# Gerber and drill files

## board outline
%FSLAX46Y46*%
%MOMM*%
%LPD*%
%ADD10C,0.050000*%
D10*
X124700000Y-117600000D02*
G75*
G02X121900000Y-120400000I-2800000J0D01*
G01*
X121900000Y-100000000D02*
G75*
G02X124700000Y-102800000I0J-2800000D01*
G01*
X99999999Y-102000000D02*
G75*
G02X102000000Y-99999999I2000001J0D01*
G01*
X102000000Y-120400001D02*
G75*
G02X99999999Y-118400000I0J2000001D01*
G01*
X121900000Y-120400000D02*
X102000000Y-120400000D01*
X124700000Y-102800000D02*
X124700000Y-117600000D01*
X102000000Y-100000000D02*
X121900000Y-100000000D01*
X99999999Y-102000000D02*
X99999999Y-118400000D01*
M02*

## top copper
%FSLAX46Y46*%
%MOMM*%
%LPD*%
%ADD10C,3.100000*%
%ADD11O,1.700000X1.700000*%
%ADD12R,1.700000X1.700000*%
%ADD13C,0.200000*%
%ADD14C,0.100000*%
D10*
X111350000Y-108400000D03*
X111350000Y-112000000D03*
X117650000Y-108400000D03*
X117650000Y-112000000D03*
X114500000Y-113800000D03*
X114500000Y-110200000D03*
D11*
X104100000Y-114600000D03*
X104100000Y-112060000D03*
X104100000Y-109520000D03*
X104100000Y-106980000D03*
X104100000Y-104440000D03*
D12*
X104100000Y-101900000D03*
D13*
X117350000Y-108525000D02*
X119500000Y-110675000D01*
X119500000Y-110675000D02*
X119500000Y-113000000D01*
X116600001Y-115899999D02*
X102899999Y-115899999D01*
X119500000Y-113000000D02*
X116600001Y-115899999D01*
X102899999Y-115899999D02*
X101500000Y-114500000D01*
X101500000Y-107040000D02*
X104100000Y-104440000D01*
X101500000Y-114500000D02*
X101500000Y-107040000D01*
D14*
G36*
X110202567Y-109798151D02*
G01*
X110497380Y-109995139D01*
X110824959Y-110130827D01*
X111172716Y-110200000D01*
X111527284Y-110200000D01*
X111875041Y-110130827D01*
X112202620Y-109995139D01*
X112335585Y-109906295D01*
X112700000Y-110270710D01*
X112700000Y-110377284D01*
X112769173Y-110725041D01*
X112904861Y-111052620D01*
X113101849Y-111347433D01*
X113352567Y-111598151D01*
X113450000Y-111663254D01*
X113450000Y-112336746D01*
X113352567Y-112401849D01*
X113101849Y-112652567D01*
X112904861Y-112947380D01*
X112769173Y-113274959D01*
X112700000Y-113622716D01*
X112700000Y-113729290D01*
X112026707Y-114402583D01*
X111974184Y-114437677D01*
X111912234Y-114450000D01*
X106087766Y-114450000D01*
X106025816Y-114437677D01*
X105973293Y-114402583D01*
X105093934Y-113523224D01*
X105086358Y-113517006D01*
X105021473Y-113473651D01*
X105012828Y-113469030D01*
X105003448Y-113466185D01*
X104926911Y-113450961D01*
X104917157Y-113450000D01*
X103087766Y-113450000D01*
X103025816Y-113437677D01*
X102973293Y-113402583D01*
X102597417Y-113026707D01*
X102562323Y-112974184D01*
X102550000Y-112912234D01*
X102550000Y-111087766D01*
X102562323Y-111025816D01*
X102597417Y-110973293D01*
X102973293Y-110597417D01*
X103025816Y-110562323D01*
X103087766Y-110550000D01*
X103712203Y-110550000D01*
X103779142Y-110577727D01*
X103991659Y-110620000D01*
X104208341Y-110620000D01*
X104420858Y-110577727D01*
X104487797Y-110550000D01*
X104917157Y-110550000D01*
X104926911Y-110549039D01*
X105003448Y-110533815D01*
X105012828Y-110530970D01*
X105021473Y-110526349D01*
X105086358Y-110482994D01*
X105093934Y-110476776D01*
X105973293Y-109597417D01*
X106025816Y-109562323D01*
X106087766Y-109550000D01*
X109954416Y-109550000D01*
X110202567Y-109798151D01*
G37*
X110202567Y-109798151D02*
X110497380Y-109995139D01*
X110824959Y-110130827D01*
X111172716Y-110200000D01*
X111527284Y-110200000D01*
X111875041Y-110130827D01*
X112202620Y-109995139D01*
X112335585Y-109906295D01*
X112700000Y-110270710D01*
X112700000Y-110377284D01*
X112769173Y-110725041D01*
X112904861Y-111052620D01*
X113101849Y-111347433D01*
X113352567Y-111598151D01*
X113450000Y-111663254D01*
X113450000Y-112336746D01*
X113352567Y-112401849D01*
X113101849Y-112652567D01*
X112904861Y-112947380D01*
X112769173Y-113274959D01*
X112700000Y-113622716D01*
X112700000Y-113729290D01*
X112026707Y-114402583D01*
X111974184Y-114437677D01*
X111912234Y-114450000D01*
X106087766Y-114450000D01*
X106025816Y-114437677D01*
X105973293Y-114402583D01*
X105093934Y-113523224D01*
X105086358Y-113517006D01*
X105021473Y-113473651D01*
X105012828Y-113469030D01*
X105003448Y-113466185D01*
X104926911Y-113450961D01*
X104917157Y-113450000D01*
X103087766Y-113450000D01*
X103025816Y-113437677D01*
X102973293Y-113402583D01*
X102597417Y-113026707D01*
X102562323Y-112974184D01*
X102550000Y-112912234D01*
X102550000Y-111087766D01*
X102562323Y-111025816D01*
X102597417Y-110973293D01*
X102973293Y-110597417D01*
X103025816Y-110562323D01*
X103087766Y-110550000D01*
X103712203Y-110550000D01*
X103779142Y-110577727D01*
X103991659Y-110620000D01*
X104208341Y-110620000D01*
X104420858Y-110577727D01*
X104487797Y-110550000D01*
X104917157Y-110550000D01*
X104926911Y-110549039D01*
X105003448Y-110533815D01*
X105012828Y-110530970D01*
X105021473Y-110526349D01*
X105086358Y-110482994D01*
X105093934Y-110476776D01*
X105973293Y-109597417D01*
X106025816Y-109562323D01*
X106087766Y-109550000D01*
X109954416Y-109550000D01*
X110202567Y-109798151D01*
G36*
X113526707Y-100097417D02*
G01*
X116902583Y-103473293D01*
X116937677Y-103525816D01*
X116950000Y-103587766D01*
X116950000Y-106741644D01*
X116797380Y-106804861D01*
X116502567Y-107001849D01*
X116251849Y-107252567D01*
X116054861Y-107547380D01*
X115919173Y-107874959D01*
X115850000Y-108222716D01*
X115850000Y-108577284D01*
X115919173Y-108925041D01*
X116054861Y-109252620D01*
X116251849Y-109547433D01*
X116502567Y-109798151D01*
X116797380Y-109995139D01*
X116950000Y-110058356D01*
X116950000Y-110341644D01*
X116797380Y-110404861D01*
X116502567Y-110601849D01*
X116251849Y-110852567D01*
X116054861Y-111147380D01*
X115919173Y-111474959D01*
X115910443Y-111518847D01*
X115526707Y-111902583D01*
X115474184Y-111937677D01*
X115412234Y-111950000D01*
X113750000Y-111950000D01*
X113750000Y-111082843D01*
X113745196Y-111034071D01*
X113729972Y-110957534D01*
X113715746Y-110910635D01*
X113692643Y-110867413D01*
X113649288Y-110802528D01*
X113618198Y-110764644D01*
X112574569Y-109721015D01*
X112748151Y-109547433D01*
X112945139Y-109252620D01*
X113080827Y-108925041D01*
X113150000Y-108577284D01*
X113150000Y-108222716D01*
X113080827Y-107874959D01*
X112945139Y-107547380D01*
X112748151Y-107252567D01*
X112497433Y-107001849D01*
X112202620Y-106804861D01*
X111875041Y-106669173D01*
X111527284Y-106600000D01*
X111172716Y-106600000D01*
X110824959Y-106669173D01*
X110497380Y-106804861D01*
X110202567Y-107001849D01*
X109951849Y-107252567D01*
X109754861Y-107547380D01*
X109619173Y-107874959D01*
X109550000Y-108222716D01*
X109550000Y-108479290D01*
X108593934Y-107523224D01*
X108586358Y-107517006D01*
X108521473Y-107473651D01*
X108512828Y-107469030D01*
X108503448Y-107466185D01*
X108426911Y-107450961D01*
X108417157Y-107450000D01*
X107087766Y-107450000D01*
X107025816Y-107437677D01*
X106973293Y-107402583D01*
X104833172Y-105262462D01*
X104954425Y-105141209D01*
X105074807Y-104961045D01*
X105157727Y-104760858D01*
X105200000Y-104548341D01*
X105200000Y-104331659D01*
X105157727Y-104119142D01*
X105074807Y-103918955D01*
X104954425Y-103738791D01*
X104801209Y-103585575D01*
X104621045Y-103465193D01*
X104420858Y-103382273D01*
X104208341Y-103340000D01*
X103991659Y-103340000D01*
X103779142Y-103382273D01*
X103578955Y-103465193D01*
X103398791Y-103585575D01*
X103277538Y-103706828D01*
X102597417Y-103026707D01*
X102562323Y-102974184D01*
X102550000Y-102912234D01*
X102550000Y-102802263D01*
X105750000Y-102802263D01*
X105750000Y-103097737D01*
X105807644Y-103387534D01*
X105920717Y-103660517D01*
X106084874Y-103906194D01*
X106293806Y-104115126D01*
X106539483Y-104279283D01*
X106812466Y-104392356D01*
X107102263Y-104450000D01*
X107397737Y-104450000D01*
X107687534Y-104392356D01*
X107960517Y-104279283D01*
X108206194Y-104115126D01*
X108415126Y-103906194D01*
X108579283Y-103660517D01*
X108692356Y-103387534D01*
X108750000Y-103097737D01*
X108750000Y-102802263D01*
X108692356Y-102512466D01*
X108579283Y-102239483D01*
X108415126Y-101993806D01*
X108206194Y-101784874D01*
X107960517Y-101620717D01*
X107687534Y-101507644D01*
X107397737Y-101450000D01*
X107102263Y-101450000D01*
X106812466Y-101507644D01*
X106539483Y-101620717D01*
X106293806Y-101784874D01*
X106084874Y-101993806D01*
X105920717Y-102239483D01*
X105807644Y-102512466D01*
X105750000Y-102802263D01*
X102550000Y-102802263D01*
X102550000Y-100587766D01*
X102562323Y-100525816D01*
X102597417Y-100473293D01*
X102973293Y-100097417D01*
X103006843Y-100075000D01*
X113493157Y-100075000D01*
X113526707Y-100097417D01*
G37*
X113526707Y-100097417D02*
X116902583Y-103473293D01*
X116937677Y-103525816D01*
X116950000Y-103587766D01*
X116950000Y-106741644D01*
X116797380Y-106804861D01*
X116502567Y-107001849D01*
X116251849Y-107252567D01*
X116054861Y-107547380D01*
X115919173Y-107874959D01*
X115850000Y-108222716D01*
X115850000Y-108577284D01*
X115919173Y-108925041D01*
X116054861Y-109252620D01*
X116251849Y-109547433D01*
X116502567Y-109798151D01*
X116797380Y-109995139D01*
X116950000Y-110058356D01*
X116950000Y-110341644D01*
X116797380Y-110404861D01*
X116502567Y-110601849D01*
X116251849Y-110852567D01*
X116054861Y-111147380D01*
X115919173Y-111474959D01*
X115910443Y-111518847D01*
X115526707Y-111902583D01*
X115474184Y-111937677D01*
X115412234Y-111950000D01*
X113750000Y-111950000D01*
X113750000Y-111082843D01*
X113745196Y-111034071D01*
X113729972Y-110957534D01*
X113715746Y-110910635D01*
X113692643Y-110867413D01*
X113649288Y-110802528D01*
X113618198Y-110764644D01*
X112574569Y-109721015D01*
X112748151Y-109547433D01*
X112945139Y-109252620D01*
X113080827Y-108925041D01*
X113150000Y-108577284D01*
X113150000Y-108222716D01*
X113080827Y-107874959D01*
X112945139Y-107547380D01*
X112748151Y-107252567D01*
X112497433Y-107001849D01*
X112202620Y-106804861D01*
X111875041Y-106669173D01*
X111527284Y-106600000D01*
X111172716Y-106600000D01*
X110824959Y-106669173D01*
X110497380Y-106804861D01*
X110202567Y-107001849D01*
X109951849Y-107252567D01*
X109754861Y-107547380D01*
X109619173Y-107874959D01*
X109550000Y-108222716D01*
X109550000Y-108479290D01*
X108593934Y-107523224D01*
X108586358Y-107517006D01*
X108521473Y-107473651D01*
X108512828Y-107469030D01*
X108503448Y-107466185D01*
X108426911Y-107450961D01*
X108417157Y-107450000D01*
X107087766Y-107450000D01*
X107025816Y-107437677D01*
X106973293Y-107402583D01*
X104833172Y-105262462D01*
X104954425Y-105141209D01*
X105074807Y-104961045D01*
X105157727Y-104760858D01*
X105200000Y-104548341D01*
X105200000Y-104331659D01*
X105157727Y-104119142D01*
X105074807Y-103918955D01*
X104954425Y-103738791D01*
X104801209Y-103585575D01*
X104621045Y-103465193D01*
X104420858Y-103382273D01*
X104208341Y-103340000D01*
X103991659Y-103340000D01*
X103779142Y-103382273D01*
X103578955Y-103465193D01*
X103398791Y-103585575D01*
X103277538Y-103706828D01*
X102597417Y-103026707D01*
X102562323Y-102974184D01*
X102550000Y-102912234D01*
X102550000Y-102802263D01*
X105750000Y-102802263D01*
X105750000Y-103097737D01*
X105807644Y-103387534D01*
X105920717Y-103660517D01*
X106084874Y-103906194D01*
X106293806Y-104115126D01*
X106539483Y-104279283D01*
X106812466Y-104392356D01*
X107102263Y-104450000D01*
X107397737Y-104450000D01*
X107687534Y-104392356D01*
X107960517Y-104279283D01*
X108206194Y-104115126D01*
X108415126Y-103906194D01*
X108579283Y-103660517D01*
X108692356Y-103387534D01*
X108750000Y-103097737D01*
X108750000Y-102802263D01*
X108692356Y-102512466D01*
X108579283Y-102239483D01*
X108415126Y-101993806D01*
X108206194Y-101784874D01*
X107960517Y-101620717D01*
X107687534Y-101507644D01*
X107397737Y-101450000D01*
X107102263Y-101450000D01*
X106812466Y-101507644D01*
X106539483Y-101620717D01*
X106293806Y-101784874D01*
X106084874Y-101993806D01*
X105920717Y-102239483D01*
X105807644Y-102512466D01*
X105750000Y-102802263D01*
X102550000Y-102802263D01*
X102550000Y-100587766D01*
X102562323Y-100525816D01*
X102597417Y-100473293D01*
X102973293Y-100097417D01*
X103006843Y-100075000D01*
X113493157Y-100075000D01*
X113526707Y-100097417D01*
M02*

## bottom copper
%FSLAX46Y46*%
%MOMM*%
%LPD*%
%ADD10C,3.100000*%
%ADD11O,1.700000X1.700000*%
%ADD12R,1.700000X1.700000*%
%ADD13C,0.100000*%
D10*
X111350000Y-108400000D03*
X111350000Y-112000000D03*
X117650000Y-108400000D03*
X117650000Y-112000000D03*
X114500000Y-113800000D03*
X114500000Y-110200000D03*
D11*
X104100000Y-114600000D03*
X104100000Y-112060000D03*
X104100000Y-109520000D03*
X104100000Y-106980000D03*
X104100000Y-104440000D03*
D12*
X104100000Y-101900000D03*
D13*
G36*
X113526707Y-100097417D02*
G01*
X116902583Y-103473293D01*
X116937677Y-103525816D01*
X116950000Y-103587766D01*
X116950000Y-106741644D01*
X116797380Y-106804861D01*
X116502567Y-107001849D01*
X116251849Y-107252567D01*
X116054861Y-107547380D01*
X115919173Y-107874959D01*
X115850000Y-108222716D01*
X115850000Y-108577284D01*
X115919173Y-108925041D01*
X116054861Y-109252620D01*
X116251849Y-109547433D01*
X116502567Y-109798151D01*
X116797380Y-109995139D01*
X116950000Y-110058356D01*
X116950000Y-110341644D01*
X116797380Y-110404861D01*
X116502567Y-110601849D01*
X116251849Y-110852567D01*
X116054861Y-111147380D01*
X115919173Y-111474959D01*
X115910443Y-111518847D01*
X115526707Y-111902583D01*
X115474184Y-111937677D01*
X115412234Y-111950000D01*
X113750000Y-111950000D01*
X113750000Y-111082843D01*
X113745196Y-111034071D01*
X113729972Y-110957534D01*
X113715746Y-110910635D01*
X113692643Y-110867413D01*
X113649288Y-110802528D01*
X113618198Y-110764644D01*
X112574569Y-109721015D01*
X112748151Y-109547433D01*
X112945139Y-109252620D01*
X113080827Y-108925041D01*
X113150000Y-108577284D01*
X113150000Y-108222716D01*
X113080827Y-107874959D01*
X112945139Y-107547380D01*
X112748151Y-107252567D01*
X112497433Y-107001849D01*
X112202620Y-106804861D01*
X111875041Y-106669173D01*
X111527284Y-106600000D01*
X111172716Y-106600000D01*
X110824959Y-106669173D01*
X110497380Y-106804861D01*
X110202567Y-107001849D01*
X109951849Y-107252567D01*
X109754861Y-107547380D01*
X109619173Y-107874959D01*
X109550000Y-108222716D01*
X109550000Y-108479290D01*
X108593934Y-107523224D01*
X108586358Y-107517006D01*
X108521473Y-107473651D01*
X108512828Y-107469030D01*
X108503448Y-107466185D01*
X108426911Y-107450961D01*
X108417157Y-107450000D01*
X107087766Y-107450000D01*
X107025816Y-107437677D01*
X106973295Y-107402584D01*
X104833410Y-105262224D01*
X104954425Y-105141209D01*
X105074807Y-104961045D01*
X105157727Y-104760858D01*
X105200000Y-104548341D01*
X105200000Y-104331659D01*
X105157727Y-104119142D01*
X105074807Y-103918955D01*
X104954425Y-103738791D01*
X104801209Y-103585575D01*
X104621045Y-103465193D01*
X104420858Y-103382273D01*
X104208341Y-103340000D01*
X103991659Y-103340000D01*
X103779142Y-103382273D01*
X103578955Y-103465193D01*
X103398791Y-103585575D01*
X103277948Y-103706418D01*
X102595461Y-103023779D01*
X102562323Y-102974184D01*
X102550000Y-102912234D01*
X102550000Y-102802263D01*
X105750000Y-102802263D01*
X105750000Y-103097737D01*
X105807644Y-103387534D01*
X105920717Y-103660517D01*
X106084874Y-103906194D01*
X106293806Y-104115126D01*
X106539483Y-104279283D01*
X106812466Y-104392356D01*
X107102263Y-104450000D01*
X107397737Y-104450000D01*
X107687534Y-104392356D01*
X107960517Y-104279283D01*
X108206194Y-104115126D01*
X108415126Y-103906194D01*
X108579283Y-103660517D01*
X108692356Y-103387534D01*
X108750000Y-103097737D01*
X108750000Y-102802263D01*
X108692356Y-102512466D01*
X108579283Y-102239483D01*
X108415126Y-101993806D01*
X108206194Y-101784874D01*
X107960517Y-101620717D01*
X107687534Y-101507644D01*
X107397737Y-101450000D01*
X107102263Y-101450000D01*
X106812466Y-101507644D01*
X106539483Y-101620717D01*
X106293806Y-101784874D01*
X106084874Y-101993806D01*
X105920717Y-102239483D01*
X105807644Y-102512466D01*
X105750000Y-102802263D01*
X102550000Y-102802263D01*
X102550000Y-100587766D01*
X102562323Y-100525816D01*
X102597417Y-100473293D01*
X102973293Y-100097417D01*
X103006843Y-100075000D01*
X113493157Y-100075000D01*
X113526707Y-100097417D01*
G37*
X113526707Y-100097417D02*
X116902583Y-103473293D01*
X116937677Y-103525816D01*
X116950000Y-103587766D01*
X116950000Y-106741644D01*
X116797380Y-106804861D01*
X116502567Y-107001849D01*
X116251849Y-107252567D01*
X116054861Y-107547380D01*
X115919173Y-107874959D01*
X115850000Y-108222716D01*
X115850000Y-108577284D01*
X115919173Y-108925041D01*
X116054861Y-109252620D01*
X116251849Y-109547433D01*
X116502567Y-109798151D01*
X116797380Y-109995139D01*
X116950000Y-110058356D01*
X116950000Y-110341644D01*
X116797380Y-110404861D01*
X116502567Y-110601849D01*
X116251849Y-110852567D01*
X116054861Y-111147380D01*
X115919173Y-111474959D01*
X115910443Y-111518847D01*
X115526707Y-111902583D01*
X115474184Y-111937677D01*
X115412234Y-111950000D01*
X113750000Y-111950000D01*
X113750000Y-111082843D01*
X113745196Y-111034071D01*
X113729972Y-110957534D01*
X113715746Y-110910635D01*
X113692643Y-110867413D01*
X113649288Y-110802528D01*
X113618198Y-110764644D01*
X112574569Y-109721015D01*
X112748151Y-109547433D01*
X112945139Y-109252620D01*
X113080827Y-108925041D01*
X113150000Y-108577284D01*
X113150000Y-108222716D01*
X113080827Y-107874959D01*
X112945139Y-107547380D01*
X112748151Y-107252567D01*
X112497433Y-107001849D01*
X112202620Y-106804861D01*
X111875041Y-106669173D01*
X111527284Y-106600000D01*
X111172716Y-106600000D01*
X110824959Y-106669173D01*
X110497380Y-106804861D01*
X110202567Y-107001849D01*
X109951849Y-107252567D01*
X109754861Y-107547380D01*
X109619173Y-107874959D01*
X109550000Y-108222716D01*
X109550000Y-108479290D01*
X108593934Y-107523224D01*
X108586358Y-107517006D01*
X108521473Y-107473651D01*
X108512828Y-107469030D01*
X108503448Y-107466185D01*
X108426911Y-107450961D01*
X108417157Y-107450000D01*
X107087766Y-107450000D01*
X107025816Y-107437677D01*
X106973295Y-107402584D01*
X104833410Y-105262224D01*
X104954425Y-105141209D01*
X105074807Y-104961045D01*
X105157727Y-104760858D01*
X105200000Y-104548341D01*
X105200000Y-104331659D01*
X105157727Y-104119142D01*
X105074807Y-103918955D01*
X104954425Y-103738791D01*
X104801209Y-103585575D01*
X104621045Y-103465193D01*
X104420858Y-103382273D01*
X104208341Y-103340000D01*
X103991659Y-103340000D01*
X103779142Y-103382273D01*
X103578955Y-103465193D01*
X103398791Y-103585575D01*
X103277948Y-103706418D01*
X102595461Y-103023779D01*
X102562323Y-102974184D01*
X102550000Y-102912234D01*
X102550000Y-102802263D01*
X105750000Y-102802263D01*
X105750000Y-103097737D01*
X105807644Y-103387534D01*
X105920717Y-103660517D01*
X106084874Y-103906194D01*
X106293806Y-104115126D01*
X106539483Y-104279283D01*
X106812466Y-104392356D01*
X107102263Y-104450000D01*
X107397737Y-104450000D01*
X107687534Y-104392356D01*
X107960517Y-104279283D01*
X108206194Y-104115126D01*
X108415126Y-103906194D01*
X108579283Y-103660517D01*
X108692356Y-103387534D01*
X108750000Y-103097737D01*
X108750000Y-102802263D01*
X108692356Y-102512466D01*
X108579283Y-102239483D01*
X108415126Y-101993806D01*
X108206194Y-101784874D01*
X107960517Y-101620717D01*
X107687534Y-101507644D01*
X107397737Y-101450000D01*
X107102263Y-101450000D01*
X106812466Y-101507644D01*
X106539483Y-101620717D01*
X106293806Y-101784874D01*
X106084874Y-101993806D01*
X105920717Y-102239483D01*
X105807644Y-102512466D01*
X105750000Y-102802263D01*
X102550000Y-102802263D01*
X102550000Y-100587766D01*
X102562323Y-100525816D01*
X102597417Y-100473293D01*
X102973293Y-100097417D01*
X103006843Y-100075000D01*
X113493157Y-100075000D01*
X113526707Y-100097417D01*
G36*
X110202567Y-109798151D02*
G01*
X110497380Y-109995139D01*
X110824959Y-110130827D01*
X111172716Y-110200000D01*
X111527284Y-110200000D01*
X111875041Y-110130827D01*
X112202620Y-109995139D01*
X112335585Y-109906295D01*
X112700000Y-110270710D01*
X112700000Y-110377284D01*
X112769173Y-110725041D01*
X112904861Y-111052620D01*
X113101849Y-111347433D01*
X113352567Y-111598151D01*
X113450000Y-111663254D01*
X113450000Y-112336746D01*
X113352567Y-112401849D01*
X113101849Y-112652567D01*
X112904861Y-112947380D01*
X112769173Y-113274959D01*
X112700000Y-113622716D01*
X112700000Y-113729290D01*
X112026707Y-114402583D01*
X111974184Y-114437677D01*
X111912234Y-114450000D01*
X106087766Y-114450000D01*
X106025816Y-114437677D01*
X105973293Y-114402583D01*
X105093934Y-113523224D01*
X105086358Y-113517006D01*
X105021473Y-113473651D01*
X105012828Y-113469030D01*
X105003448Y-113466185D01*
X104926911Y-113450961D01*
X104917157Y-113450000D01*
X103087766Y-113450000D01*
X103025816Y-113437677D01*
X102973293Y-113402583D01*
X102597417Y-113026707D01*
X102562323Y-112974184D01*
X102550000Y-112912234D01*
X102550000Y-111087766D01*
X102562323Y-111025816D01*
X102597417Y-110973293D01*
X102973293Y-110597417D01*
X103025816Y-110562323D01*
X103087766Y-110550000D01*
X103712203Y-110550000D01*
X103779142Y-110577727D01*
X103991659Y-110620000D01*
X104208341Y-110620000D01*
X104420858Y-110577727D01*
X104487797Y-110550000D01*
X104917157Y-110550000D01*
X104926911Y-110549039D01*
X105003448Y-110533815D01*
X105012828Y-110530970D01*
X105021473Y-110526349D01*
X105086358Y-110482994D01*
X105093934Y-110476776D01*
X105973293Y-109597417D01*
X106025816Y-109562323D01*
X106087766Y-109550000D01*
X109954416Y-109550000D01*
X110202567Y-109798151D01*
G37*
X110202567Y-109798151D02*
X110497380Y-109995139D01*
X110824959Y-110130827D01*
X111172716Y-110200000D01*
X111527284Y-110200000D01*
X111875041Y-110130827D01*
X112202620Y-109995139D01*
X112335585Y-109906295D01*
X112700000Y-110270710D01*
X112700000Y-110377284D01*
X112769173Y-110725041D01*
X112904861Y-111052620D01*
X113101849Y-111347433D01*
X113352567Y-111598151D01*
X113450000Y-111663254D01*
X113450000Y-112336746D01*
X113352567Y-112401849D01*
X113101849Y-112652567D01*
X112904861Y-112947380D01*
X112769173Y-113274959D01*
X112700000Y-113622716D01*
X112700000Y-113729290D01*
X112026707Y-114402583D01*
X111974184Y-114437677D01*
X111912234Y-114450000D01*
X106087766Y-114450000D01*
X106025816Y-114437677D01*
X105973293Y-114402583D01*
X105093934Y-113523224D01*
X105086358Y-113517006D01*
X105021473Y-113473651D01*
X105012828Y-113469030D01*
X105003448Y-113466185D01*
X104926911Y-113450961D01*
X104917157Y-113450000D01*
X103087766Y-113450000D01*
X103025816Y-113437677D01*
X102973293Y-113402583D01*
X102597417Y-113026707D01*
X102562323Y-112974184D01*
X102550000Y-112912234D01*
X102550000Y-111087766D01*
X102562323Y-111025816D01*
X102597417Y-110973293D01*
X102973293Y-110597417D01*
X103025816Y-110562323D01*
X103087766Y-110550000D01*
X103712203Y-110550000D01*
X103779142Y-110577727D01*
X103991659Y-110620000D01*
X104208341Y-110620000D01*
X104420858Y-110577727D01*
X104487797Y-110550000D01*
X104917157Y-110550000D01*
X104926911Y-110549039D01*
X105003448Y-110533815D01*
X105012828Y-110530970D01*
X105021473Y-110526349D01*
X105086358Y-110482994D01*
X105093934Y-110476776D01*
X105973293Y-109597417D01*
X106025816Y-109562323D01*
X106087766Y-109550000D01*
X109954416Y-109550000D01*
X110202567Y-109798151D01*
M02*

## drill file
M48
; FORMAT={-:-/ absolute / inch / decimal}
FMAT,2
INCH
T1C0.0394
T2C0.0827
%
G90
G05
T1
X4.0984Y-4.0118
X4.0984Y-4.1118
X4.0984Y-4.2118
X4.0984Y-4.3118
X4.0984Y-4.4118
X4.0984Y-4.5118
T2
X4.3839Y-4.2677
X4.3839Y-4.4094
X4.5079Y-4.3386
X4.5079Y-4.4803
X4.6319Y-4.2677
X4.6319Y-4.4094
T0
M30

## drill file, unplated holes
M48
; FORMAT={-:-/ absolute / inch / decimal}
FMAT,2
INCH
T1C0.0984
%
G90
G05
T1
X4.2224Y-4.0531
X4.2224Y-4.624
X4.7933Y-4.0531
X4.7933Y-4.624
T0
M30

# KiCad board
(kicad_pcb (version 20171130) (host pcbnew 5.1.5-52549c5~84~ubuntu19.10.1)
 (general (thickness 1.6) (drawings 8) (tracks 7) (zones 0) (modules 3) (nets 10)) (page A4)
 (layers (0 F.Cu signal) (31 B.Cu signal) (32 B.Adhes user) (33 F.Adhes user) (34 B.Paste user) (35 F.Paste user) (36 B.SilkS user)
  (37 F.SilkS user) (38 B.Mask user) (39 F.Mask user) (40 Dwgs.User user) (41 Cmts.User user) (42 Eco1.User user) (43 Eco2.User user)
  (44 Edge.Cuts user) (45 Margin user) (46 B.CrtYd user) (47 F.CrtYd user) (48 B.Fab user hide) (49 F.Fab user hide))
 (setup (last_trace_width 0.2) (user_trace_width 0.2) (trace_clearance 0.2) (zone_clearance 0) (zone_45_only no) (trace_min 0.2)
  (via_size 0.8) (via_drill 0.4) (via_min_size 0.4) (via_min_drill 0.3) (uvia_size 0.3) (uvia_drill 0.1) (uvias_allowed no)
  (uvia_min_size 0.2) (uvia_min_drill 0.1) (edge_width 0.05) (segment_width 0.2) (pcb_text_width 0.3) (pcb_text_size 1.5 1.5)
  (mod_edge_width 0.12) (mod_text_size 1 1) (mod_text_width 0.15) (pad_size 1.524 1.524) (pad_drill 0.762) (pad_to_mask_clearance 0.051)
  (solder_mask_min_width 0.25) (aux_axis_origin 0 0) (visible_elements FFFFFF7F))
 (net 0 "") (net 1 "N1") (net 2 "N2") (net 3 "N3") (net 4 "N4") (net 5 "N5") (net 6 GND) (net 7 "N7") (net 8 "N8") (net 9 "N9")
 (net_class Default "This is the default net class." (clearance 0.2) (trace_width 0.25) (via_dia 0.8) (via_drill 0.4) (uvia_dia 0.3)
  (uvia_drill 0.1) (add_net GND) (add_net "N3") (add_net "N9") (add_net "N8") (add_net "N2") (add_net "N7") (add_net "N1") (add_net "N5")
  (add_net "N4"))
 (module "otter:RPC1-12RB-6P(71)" (layer F.Cu) (at 114.5 110.2 270)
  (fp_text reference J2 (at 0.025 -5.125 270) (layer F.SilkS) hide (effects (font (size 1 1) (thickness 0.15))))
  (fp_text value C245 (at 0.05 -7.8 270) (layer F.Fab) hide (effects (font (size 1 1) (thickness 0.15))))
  (pad "" np_thru_hole circle (at -7.25 -7.25 270) (size 2.5 2.5) (drill 2.5) (layers *.Cu *.Mask))
  (pad "" np_thru_hole circle (at -7.25 7.25 270) (size 2.5 2.5) (drill 2.5) (layers *.Cu *.Mask))
  (pad "" np_thru_hole circle (at 7.25 7.25 270) (size 2.5 2.5) (drill 2.5) (layers *.Cu *.Mask))
  (pad "" np_thru_hole circle (at 7.25 -7.25 270) (size 2.5 2.5) (drill 2.5) (layers *.Cu *.Mask))
  (pad 1 thru_hole circle (at -1.8 3.15 270) (size 3.1 3.1) (drill 2.1) (layers *.Cu *.Mask) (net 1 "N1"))
  (pad 2 thru_hole circle (at 1.8 3.15 270) (size 3.1 3.1) (drill 2.1) (layers *.Cu *.Mask) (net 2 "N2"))
  (pad 5 thru_hole circle (at -1.8 -3.15 270) (size 3.1 3.1) (drill 2.1) (layers *.Cu *.Mask) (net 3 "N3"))
  (pad 4 thru_hole circle (at 1.8 -3.15 270) (size 3.1 3.1) (drill 2.1) (layers *.Cu *.Mask) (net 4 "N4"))
  (pad 3 thru_hole circle (at 3.6 0 270) (size 3.1 3.1) (drill 2.1) (layers *.Cu *.Mask) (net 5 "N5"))
  (pad 6 thru_hole circle (at 0 0 270) (size 3.1 3.1) (drill 2.1) (layers *.Cu *.Mask) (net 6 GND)))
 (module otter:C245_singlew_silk (layer F.Cu) (at 101.7 110.2 270)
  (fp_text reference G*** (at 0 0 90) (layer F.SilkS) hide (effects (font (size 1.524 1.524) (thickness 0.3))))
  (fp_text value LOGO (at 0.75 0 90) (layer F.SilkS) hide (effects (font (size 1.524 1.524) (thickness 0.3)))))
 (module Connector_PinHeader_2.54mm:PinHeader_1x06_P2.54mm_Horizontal (layer B.Cu) (at 104.1 101.9 180)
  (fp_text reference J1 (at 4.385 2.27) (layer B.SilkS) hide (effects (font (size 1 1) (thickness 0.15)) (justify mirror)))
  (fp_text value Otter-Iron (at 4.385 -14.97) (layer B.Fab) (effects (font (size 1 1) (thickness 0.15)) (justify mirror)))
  (pad 6 thru_hole oval (at 0 -12.7 180) (size 1.7 1.7) (drill 1) (layers *.Cu *.Mask) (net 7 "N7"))
  (pad 5 thru_hole oval (at 0 -10.16 180) (size 1.7 1.7) (drill 1) (layers *.Cu *.Mask) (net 2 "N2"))
  (pad 4 thru_hole oval (at 0 -7.62 180) (size 1.7 1.7) (drill 1) (layers *.Cu *.Mask) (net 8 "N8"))
  (pad 3 thru_hole oval (at 0 -5.08 180) (size 1.7 1.7) (drill 1) (layers *.Cu *.Mask) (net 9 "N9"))
  (pad 2 thru_hole oval (at 0 -2.54 180) (size 1.7 1.7) (drill 1) (layers *.Cu *.Mask) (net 3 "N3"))
  (pad 1 thru_hole rect (at 0 0 180) (size 1.7 1.7) (drill 1) (layers *.Cu *.Mask) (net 6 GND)))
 (gr_arc (start 121.9 117.6) (end 121.9 120.4) (angle -90) (layer Edge.Cuts) (width 0.05))
 (gr_arc (start 121.9 102.8) (end 124.7 102.8) (angle -90) (layer Edge.Cuts) (width 0.05))
 (gr_arc (start 102 102) (end 102 99.999999) (angle -90) (layer Edge.Cuts) (width 0.05))
 (gr_arc (start 102 118.4) (end 99.999999 118.4) (angle -90) (layer Edge.Cuts) (width 0.05))
 (gr_line (start 121.9 120.4) (end 102 120.4) (layer Edge.Cuts) (width 0.05))
 (gr_line (start 124.7 102.8) (end 124.7 117.6) (layer Edge.Cuts) (width 0.05))
 (gr_line (start 102 100) (end 121.9 100) (layer Edge.Cuts) (width 0.05))
 (gr_line (start 99.999999 102) (end 99.999999 118.4) (layer Edge.Cuts) (width 0.05))
 (segment (start 117.35 108.525) (end 119.5 110.675) (width 0.2) (layer F.Cu) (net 3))
 (segment (start 119.5 110.675) (end 119.5 113) (width 0.2) (layer F.Cu) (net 3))
 (segment (start 116.600001 115.899999) (end 102.899999 115.899999) (width 0.2) (layer F.Cu) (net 3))
 (segment (start 119.5 113) (end 116.600001 115.899999) (width 0.2) (layer F.Cu) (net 3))
 (segment (start 102.899999 115.899999) (end 101.5 114.5) (width 0.2) (layer F.Cu) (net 3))
 (segment (start 101.5 107.04) (end 104.1 104.44) (width 0.2) (layer F.Cu) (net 3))
 (segment (start 101.5 114.5) (end 101.5 107.04) (width 0.2) (layer F.Cu) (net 3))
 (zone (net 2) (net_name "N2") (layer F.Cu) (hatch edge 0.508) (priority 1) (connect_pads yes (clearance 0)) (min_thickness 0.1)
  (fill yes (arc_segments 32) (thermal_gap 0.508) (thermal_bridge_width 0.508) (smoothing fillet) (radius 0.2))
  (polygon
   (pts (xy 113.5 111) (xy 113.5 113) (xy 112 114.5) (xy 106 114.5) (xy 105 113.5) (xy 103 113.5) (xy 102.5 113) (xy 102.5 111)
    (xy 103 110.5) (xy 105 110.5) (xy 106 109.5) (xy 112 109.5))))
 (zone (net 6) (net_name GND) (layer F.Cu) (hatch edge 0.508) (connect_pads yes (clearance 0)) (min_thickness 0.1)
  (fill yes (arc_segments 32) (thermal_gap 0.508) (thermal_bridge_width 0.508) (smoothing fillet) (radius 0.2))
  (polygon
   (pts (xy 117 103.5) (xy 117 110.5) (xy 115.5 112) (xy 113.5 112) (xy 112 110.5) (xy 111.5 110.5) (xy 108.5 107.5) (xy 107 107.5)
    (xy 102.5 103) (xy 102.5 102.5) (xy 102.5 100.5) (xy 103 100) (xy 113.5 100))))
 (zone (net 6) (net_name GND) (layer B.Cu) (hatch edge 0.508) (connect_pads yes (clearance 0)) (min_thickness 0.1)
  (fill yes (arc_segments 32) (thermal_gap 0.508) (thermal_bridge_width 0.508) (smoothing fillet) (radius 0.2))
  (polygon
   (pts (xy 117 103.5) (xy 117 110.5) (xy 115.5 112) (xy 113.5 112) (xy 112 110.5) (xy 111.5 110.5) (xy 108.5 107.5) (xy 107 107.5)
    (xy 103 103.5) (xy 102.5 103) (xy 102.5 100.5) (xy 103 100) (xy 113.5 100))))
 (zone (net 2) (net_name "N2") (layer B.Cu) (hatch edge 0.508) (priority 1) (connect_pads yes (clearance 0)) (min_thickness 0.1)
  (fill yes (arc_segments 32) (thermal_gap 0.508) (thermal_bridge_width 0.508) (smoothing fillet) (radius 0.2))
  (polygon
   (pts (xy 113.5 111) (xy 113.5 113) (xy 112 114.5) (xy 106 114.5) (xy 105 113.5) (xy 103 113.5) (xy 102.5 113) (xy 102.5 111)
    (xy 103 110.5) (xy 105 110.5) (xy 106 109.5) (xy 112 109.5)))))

